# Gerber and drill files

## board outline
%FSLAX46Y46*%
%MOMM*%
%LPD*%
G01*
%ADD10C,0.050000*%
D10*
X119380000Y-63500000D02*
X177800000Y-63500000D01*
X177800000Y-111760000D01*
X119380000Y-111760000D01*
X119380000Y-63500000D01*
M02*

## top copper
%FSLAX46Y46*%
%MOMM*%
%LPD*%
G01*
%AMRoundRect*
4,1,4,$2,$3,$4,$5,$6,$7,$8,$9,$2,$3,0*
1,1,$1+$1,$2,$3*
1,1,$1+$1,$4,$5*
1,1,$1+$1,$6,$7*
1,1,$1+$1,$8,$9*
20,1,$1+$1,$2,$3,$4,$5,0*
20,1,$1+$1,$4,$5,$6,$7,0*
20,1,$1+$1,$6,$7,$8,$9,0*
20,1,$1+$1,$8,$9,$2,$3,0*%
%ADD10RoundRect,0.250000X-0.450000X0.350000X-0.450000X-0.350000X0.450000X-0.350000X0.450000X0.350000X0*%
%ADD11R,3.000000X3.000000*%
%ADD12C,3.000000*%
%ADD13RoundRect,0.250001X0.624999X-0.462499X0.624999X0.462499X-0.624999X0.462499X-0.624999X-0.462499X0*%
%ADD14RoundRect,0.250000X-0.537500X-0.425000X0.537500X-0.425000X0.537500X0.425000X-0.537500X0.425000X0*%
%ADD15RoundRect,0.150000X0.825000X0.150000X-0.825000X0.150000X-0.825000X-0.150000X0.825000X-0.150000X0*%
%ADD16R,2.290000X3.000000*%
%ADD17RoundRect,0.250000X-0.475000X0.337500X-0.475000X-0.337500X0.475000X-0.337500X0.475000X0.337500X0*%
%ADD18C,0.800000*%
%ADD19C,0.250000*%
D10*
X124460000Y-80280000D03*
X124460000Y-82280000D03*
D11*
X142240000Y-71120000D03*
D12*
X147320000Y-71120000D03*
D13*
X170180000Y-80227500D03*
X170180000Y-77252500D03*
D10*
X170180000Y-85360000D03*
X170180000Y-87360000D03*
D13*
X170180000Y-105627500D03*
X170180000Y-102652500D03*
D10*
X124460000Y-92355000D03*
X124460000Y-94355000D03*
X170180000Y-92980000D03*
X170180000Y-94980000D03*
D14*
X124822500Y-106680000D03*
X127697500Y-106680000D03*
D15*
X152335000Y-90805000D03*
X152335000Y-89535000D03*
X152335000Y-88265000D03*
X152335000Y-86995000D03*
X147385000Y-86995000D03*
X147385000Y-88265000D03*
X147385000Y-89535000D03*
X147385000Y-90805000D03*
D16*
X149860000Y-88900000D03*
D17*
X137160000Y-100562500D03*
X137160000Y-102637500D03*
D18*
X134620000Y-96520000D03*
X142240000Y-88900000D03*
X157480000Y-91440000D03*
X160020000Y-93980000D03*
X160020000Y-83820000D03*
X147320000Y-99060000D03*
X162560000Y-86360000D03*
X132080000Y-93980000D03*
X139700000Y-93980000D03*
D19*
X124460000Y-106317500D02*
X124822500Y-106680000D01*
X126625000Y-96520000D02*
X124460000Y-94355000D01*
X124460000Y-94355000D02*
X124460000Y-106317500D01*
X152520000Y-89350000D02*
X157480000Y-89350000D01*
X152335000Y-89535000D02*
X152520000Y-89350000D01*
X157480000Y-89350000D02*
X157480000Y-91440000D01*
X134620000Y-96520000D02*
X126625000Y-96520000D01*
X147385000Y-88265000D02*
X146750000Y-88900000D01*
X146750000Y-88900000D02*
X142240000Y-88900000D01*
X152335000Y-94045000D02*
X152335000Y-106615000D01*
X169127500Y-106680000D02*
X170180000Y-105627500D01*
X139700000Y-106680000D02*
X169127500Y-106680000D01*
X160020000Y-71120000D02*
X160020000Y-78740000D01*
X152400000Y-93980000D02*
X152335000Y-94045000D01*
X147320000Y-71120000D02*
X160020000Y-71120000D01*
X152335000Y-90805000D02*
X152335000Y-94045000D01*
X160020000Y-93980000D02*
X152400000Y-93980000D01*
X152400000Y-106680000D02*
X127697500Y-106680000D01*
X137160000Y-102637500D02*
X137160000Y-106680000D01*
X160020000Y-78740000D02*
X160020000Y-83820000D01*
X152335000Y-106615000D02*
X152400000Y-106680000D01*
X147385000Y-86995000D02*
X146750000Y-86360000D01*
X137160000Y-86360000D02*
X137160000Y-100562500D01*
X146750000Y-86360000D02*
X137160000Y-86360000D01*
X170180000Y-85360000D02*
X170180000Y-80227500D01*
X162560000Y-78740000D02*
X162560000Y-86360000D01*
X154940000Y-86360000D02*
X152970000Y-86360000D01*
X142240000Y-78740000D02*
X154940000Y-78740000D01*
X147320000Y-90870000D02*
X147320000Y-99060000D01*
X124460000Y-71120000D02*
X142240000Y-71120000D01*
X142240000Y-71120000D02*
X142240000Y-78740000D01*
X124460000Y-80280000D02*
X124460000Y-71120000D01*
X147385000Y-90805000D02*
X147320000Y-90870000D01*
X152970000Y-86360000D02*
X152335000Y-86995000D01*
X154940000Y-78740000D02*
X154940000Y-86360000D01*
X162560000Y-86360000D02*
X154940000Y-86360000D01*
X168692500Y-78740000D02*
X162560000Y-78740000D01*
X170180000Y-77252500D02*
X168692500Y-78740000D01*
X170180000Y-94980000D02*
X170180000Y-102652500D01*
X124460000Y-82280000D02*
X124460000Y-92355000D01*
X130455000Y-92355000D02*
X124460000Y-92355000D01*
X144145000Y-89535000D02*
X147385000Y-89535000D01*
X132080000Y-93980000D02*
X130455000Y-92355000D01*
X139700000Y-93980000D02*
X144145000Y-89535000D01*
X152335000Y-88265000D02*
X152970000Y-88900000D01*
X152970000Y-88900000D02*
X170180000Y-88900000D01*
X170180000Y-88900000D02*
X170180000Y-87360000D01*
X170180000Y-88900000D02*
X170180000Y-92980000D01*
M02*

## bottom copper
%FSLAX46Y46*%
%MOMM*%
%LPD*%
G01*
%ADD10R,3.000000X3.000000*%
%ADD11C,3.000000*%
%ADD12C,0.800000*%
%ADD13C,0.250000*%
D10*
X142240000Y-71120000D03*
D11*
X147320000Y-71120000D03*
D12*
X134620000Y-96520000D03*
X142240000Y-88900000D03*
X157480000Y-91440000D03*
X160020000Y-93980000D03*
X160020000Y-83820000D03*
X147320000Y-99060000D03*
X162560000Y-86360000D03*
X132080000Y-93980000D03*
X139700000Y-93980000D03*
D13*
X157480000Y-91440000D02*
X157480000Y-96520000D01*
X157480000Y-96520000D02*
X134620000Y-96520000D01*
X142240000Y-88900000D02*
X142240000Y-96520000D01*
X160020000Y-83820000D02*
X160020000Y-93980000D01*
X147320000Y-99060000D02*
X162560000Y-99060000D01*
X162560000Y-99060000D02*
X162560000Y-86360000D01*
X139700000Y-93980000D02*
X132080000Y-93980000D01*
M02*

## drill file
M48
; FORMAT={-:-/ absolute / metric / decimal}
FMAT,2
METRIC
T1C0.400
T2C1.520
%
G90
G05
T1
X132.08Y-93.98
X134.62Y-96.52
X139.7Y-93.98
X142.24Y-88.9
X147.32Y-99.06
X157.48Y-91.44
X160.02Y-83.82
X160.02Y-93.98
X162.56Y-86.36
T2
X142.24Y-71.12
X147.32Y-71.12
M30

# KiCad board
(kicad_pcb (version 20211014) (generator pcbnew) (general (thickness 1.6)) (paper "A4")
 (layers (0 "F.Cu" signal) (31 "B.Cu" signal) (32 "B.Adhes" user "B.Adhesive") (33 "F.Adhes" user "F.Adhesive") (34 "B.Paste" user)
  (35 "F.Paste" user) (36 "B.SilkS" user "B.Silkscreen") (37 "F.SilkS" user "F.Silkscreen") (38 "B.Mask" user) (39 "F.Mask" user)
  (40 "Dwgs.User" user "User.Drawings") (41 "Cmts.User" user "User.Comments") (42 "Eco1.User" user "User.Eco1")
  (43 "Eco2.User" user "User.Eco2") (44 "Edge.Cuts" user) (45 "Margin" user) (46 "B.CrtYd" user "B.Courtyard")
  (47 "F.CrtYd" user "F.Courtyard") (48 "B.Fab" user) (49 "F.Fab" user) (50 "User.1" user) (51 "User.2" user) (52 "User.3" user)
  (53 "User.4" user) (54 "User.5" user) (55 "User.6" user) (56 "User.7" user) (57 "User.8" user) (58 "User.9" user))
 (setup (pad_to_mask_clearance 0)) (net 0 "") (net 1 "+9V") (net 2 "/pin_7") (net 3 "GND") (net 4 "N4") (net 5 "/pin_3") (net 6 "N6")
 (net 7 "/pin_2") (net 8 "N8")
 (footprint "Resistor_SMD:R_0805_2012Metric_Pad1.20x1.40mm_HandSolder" (layer "F.Cu") (at 124.46 81.28 -90)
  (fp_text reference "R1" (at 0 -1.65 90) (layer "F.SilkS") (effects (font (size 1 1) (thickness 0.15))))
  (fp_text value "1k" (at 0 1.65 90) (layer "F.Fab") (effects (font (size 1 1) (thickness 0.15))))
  (pad "1" smd roundrect (at -1 0 270) (size 1.2 1.4) (layers "F.Cu" "F.Paste" "F.Mask") (roundrect_rratio 0.208333) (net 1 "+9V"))
  (pad "2" smd roundrect (at 1 0 270) (size 1.2 1.4) (layers "F.Cu" "F.Paste" "F.Mask") (roundrect_rratio 0.208333) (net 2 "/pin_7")))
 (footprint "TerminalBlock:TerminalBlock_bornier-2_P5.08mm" (layer "F.Cu") (at 142.24 71.12)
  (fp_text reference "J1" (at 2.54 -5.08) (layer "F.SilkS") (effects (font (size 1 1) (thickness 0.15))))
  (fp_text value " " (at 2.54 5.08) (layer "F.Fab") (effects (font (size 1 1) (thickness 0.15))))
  (pad "1" thru_hole rect (at 0 0) (size 3 3) (drill 1.52) (layers *.Cu *.Mask) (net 1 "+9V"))
  (pad "2" thru_hole circle (at 5.08 0) (size 3 3) (drill 1.52) (layers *.Cu *.Mask) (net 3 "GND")))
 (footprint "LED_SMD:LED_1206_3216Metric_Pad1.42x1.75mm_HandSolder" (layer "F.Cu") (at 170.18 78.74 90)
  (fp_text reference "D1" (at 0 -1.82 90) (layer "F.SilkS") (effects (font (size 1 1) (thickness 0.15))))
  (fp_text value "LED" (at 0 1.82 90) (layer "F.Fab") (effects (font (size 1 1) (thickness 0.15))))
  (pad "1" smd roundrect (at -1.4875 0 90) (size 1.425 1.75) (layers "F.Cu" "F.Paste" "F.Mask") (roundrect_rratio 0.175439) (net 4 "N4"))
  (pad "2" smd roundrect (at 1.4875 0 90) (size 1.425 1.75) (layers "F.Cu" "F.Paste" "F.Mask") (roundrect_rratio 0.175439) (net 1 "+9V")))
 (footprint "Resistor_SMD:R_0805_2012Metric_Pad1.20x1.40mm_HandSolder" (layer "F.Cu") (at 170.18 86.36 -90)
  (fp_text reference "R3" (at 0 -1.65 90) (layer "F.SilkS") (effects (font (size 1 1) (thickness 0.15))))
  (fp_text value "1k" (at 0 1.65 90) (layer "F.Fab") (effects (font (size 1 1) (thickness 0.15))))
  (pad "1" smd roundrect (at -1 0 270) (size 1.2 1.4) (layers "F.Cu" "F.Paste" "F.Mask") (roundrect_rratio 0.208333) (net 4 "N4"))
  (pad "2" smd roundrect (at 1 0 270) (size 1.2 1.4) (layers "F.Cu" "F.Paste" "F.Mask") (roundrect_rratio 0.208333) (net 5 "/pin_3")))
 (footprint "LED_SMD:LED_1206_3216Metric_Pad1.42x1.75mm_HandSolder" (layer "F.Cu") (at 170.18 104.14 90)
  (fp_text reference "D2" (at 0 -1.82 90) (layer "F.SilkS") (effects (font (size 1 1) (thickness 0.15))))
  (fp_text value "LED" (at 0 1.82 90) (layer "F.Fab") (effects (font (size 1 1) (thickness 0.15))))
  (pad "1" smd roundrect (at -1.4875 0 90) (size 1.425 1.75) (layers "F.Cu" "F.Paste" "F.Mask") (roundrect_rratio 0.175439) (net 3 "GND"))
  (pad "2" smd roundrect (at 1.4875 0 90) (size 1.425 1.75) (layers "F.Cu" "F.Paste" "F.Mask") (roundrect_rratio 0.175439) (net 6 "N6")))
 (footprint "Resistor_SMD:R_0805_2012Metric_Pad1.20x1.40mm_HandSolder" (layer "F.Cu") (at 124.46 93.355 -90)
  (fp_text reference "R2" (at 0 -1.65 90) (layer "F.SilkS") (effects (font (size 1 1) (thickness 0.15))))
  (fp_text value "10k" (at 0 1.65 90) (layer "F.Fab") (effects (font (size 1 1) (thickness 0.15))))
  (pad "1" smd roundrect (at -1 0 270) (size 1.2 1.4) (layers "F.Cu" "F.Paste" "F.Mask") (roundrect_rratio 0.208333) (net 2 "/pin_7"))
  (pad "2" smd roundrect (at 1 0 270) (size 1.2 1.4) (layers "F.Cu" "F.Paste" "F.Mask") (roundrect_rratio 0.208333) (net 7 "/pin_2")))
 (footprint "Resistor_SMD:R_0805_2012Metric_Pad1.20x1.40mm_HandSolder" (layer "F.Cu") (at 170.18 93.98 -90)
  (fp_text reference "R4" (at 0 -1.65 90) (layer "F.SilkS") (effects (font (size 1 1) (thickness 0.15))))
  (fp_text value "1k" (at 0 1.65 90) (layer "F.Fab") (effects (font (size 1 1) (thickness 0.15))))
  (pad "1" smd roundrect (at -1 0 270) (size 1.2 1.4) (layers "F.Cu" "F.Paste" "F.Mask") (roundrect_rratio 0.208333) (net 5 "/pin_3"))
  (pad "2" smd roundrect (at 1 0 270) (size 1.2 1.4) (layers "F.Cu" "F.Paste" "F.Mask") (roundrect_rratio 0.208333) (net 6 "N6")))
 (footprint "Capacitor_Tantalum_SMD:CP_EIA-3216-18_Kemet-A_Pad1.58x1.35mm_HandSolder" (layer "F.Cu") (at 126.26 106.68)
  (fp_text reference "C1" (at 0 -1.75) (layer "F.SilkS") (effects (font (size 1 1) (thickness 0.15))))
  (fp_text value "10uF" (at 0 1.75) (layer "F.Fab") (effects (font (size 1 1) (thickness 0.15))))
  (pad "1" smd roundrect (at -1.4375 0) (size 1.575 1.35) (layers "F.Cu" "F.Paste" "F.Mask") (roundrect_rratio 0.185185) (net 7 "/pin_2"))
  (pad "2" smd roundrect (at 1.4375 0) (size 1.575 1.35) (layers "F.Cu" "F.Paste" "F.Mask") (roundrect_rratio 0.185185) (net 3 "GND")))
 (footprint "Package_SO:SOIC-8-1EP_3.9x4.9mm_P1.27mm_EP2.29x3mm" (layer "F.Cu") (at 149.86 88.9 180)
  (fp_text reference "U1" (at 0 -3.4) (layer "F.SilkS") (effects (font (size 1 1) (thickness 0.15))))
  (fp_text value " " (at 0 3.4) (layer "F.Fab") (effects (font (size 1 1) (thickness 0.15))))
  (pad "" smd roundrect (at -0.57 -0.75 180) (size 0.92 1.21) (layers "F.Paste") (roundrect_rratio 0.25))
  (pad "" smd roundrect (at 0.57 0.75 180) (size 0.92 1.21) (layers "F.Paste") (roundrect_rratio 0.25))
  (pad "" smd roundrect (at -0.57 0.75 180) (size 0.92 1.21) (layers "F.Paste") (roundrect_rratio 0.25))
  (pad "" smd roundrect (at 0.57 -0.75 180) (size 0.92 1.21) (layers "F.Paste") (roundrect_rratio 0.25))
  (pad "1" smd roundrect (at -2.475 -1.905 180) (size 1.95 0.6) (layers "F.Cu" "F.Paste" "F.Mask") (roundrect_rratio 0.25) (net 3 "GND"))
  (pad "2" smd roundrect (at -2.475 -0.635 180) (size 1.95 0.6) (layers "F.Cu" "F.Paste" "F.Mask") (roundrect_rratio 0.25) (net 7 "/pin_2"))
  (pad "3" smd roundrect (at -2.475 0.635 180) (size 1.95 0.6) (layers "F.Cu" "F.Paste" "F.Mask") (roundrect_rratio 0.25) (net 5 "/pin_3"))
  (pad "4" smd roundrect (at -2.475 1.905 180) (size 1.95 0.6) (layers "F.Cu" "F.Paste" "F.Mask") (roundrect_rratio 0.25) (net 1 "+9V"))
  (pad "5" smd roundrect (at 2.475 1.905 180) (size 1.95 0.6) (layers "F.Cu" "F.Paste" "F.Mask") (roundrect_rratio 0.25) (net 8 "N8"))
  (pad "6" smd roundrect (at 2.475 0.635 180) (size 1.95 0.6) (layers "F.Cu" "F.Paste" "F.Mask") (roundrect_rratio 0.25) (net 7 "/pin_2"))
  (pad "7" smd roundrect (at 2.475 -0.635 180) (size 1.95 0.6) (layers "F.Cu" "F.Paste" "F.Mask") (roundrect_rratio 0.25) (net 2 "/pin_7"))
  (pad "8" smd roundrect (at 2.475 -1.905 180) (size 1.95 0.6) (layers "F.Cu" "F.Paste" "F.Mask") (roundrect_rratio 0.25) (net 1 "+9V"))
  (pad "9" smd rect (at 0 0 180) (size 2.29 3) (layers "F.Cu" "F.Mask")))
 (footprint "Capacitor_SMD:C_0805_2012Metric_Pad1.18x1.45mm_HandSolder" (layer "F.Cu") (at 137.16 101.6 -90)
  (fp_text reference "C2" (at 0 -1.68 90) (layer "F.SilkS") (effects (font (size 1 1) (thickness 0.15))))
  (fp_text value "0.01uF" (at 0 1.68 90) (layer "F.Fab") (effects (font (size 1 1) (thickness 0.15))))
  (pad "1" smd roundrect (at -1.0375 0 270) (size 1.175 1.45) (layers "F.Cu" "F.Paste" "F.Mask") (roundrect_rratio 0.212766) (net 8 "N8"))
  (pad "2" smd roundrect (at 1.0375 0 270) (size 1.175 1.45) (layers "F.Cu" "F.Paste" "F.Mask") (roundrect_rratio 0.212766) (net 3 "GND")))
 (gr_rect (start 119.38 63.5) (end 177.8 111.76) (layer "Edge.Cuts") (width 0.05) (fill none))
 (segment (start 124.46 106.3175) (end 124.8225 106.68) (width 0.25) (layer "F.Cu") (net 7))
 (segment (start 126.625 96.52) (end 124.46 94.355) (width 0.25) (layer "F.Cu") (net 7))
 (segment (start 124.46 94.355) (end 124.46 106.3175) (width 0.25) (layer "F.Cu") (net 7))
 (segment (start 152.52 89.35) (end 157.48 89.35) (width 0.25) (layer "F.Cu") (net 7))
 (segment (start 152.335 89.535) (end 152.52 89.35) (width 0.25) (layer "F.Cu") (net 7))
 (segment (start 157.48 89.35) (end 157.48 91.44) (width 0.25) (layer "F.Cu") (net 7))
 (segment (start 134.62 96.52) (end 126.625 96.52) (width 0.25) (layer "F.Cu") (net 7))
 (segment (start 147.385 88.265) (end 146.75 88.9) (width 0.25) (layer "F.Cu") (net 7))
 (segment (start 146.75 88.9) (end 142.24 88.9) (width 0.25) (layer "F.Cu") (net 7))
 (via (at 134.62 96.52) (size 0.8) (drill 0.4) (layers "F.Cu" "B.Cu") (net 7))
 (via (at 142.24 88.9) (size 0.8) (drill 0.4) (layers "F.Cu" "B.Cu") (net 7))
 (via (at 157.48 91.44) (size 0.8) (drill 0.4) (layers "F.Cu" "B.Cu") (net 7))
 (segment (start 157.48 91.44) (end 157.48 96.52) (width 0.25) (layer "B.Cu") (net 7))
 (segment (start 157.48 96.52) (end 134.62 96.52) (width 0.25) (layer "B.Cu") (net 7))
 (segment (start 142.24 88.9) (end 142.24 96.52) (width 0.25) (layer "B.Cu") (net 7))
 (segment (start 152.335 94.045) (end 152.335 106.615) (width 0.25) (layer "F.Cu") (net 3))
 (segment (start 169.1275 106.68) (end 170.18 105.6275) (width 0.25) (layer "F.Cu") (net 3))
 (segment (start 139.7 106.68) (end 169.1275 106.68) (width 0.25) (layer "F.Cu") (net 3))
 (segment (start 160.02 71.12) (end 160.02 78.74) (width 0.25) (layer "F.Cu") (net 3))
 (segment (start 152.4 93.98) (end 152.335 94.045) (width 0.25) (layer "F.Cu") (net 3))
 (segment (start 147.32 71.12) (end 160.02 71.12) (width 0.25) (layer "F.Cu") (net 3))
 (segment (start 152.335 90.805) (end 152.335 94.045) (width 0.25) (layer "F.Cu") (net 3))
 (segment (start 160.02 93.98) (end 152.4 93.98) (width 0.25) (layer "F.Cu") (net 3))
 (segment (start 152.4 106.68) (end 127.6975 106.68) (width 0.25) (layer "F.Cu") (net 3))
 (segment (start 137.16 102.6375) (end 137.16 106.68) (width 0.25) (layer "F.Cu") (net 3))
 (segment (start 160.02 78.74) (end 160.02 83.82) (width 0.25) (layer "F.Cu") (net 3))
 (segment (start 152.335 106.615) (end 152.4 106.68) (width 0.25) (layer "F.Cu") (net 3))
 (via (at 160.02 93.98) (size 0.8) (drill 0.4) (layers "F.Cu" "B.Cu") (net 3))
 (via (at 160.02 83.82) (size 0.8) (drill 0.4) (layers "F.Cu" "B.Cu") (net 3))
 (segment (start 160.02 83.82) (end 160.02 93.98) (width 0.25) (layer "B.Cu") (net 3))
 (segment (start 147.385 86.995) (end 146.75 86.36) (width 0.25) (layer "F.Cu") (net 8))
 (segment (start 137.16 86.36) (end 137.16 100.5625) (width 0.25) (layer "F.Cu") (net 8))
 (segment (start 146.75 86.36) (end 137.16 86.36) (width 0.25) (layer "F.Cu") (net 8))
 (segment (start 170.18 85.36) (end 170.18 80.2275) (width 0.25) (layer "F.Cu") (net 4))
 (segment (start 162.56 78.74) (end 162.56 86.36) (width 0.25) (layer "F.Cu") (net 1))
 (segment (start 154.94 86.36) (end 152.97 86.36) (width 0.25) (layer "F.Cu") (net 1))
 (segment (start 142.24 78.74) (end 154.94 78.74) (width 0.25) (layer "F.Cu") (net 1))
 (segment (start 147.32 90.87) (end 147.32 99.06) (width 0.25) (layer "F.Cu") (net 1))
 (segment (start 124.46 71.12) (end 142.24 71.12) (width 0.25) (layer "F.Cu") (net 1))
 (segment (start 142.24 71.12) (end 142.24 78.74) (width 0.25) (layer "F.Cu") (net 1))
 (segment (start 124.46 80.28) (end 124.46 71.12) (width 0.25) (layer "F.Cu") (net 1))
 (segment (start 147.385 90.805) (end 147.32 90.87) (width 0.25) (layer "F.Cu") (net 1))
 (segment (start 152.97 86.36) (end 152.335 86.995) (width 0.25) (layer "F.Cu") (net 1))
 (segment (start 154.94 78.74) (end 154.94 86.36) (width 0.25) (layer "F.Cu") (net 1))
 (segment (start 162.56 86.36) (end 154.94 86.36) (width 0.25) (layer "F.Cu") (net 1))
 (segment (start 168.6925 78.74) (end 162.56 78.74) (width 0.25) (layer "F.Cu") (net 1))
 (segment (start 170.18 77.2525) (end 168.6925 78.74) (width 0.25) (layer "F.Cu") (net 1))
 (via (at 147.32 99.06) (size 0.8) (drill 0.4) (layers "F.Cu" "B.Cu") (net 1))
 (via (at 162.56 86.36) (size 0.8) (drill 0.4) (layers "F.Cu" "B.Cu") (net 1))
 (segment (start 147.32 99.06) (end 162.56 99.06) (width 0.25) (layer "B.Cu") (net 1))
 (segment (start 162.56 99.06) (end 162.56 86.36) (width 0.25) (layer "B.Cu") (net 1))
 (segment (start 170.18 94.98) (end 170.18 102.6525) (width 0.25) (layer "F.Cu") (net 6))
 (segment (start 124.46 82.28) (end 124.46 92.355) (width 0.25) (layer "F.Cu") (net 2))
 (segment (start 130.455 92.355) (end 124.46 92.355) (width 0.25) (layer "F.Cu") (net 2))
 (segment (start 144.145 89.535) (end 147.385 89.535) (width 0.25) (layer "F.Cu") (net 2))
 (segment (start 132.08 93.98) (end 130.455 92.355) (width 0.25) (layer "F.Cu") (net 2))
 (segment (start 139.7 93.98) (end 144.145 89.535) (width 0.25) (layer "F.Cu") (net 2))
 (via (at 132.08 93.98) (size 0.8) (drill 0.4) (layers "F.Cu" "B.Cu") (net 2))
 (via (at 139.7 93.98) (size 0.8) (drill 0.4) (layers "F.Cu" "B.Cu") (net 2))
 (segment (start 139.7 93.98) (end 132.08 93.98) (width 0.25) (layer "B.Cu") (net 2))
 (segment (start 152.335 88.265) (end 152.97 88.9) (width 0.25) (layer "F.Cu") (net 5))
 (segment (start 152.97 88.9) (end 170.18 88.9) (width 0.25) (layer "F.Cu") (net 5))
 (segment (start 170.18 88.9) (end 170.18 87.36) (width 0.25) (layer "F.Cu") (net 5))
 (segment (start 170.18 88.9) (end 170.18 92.98) (width 0.25) (layer "F.Cu") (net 5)))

